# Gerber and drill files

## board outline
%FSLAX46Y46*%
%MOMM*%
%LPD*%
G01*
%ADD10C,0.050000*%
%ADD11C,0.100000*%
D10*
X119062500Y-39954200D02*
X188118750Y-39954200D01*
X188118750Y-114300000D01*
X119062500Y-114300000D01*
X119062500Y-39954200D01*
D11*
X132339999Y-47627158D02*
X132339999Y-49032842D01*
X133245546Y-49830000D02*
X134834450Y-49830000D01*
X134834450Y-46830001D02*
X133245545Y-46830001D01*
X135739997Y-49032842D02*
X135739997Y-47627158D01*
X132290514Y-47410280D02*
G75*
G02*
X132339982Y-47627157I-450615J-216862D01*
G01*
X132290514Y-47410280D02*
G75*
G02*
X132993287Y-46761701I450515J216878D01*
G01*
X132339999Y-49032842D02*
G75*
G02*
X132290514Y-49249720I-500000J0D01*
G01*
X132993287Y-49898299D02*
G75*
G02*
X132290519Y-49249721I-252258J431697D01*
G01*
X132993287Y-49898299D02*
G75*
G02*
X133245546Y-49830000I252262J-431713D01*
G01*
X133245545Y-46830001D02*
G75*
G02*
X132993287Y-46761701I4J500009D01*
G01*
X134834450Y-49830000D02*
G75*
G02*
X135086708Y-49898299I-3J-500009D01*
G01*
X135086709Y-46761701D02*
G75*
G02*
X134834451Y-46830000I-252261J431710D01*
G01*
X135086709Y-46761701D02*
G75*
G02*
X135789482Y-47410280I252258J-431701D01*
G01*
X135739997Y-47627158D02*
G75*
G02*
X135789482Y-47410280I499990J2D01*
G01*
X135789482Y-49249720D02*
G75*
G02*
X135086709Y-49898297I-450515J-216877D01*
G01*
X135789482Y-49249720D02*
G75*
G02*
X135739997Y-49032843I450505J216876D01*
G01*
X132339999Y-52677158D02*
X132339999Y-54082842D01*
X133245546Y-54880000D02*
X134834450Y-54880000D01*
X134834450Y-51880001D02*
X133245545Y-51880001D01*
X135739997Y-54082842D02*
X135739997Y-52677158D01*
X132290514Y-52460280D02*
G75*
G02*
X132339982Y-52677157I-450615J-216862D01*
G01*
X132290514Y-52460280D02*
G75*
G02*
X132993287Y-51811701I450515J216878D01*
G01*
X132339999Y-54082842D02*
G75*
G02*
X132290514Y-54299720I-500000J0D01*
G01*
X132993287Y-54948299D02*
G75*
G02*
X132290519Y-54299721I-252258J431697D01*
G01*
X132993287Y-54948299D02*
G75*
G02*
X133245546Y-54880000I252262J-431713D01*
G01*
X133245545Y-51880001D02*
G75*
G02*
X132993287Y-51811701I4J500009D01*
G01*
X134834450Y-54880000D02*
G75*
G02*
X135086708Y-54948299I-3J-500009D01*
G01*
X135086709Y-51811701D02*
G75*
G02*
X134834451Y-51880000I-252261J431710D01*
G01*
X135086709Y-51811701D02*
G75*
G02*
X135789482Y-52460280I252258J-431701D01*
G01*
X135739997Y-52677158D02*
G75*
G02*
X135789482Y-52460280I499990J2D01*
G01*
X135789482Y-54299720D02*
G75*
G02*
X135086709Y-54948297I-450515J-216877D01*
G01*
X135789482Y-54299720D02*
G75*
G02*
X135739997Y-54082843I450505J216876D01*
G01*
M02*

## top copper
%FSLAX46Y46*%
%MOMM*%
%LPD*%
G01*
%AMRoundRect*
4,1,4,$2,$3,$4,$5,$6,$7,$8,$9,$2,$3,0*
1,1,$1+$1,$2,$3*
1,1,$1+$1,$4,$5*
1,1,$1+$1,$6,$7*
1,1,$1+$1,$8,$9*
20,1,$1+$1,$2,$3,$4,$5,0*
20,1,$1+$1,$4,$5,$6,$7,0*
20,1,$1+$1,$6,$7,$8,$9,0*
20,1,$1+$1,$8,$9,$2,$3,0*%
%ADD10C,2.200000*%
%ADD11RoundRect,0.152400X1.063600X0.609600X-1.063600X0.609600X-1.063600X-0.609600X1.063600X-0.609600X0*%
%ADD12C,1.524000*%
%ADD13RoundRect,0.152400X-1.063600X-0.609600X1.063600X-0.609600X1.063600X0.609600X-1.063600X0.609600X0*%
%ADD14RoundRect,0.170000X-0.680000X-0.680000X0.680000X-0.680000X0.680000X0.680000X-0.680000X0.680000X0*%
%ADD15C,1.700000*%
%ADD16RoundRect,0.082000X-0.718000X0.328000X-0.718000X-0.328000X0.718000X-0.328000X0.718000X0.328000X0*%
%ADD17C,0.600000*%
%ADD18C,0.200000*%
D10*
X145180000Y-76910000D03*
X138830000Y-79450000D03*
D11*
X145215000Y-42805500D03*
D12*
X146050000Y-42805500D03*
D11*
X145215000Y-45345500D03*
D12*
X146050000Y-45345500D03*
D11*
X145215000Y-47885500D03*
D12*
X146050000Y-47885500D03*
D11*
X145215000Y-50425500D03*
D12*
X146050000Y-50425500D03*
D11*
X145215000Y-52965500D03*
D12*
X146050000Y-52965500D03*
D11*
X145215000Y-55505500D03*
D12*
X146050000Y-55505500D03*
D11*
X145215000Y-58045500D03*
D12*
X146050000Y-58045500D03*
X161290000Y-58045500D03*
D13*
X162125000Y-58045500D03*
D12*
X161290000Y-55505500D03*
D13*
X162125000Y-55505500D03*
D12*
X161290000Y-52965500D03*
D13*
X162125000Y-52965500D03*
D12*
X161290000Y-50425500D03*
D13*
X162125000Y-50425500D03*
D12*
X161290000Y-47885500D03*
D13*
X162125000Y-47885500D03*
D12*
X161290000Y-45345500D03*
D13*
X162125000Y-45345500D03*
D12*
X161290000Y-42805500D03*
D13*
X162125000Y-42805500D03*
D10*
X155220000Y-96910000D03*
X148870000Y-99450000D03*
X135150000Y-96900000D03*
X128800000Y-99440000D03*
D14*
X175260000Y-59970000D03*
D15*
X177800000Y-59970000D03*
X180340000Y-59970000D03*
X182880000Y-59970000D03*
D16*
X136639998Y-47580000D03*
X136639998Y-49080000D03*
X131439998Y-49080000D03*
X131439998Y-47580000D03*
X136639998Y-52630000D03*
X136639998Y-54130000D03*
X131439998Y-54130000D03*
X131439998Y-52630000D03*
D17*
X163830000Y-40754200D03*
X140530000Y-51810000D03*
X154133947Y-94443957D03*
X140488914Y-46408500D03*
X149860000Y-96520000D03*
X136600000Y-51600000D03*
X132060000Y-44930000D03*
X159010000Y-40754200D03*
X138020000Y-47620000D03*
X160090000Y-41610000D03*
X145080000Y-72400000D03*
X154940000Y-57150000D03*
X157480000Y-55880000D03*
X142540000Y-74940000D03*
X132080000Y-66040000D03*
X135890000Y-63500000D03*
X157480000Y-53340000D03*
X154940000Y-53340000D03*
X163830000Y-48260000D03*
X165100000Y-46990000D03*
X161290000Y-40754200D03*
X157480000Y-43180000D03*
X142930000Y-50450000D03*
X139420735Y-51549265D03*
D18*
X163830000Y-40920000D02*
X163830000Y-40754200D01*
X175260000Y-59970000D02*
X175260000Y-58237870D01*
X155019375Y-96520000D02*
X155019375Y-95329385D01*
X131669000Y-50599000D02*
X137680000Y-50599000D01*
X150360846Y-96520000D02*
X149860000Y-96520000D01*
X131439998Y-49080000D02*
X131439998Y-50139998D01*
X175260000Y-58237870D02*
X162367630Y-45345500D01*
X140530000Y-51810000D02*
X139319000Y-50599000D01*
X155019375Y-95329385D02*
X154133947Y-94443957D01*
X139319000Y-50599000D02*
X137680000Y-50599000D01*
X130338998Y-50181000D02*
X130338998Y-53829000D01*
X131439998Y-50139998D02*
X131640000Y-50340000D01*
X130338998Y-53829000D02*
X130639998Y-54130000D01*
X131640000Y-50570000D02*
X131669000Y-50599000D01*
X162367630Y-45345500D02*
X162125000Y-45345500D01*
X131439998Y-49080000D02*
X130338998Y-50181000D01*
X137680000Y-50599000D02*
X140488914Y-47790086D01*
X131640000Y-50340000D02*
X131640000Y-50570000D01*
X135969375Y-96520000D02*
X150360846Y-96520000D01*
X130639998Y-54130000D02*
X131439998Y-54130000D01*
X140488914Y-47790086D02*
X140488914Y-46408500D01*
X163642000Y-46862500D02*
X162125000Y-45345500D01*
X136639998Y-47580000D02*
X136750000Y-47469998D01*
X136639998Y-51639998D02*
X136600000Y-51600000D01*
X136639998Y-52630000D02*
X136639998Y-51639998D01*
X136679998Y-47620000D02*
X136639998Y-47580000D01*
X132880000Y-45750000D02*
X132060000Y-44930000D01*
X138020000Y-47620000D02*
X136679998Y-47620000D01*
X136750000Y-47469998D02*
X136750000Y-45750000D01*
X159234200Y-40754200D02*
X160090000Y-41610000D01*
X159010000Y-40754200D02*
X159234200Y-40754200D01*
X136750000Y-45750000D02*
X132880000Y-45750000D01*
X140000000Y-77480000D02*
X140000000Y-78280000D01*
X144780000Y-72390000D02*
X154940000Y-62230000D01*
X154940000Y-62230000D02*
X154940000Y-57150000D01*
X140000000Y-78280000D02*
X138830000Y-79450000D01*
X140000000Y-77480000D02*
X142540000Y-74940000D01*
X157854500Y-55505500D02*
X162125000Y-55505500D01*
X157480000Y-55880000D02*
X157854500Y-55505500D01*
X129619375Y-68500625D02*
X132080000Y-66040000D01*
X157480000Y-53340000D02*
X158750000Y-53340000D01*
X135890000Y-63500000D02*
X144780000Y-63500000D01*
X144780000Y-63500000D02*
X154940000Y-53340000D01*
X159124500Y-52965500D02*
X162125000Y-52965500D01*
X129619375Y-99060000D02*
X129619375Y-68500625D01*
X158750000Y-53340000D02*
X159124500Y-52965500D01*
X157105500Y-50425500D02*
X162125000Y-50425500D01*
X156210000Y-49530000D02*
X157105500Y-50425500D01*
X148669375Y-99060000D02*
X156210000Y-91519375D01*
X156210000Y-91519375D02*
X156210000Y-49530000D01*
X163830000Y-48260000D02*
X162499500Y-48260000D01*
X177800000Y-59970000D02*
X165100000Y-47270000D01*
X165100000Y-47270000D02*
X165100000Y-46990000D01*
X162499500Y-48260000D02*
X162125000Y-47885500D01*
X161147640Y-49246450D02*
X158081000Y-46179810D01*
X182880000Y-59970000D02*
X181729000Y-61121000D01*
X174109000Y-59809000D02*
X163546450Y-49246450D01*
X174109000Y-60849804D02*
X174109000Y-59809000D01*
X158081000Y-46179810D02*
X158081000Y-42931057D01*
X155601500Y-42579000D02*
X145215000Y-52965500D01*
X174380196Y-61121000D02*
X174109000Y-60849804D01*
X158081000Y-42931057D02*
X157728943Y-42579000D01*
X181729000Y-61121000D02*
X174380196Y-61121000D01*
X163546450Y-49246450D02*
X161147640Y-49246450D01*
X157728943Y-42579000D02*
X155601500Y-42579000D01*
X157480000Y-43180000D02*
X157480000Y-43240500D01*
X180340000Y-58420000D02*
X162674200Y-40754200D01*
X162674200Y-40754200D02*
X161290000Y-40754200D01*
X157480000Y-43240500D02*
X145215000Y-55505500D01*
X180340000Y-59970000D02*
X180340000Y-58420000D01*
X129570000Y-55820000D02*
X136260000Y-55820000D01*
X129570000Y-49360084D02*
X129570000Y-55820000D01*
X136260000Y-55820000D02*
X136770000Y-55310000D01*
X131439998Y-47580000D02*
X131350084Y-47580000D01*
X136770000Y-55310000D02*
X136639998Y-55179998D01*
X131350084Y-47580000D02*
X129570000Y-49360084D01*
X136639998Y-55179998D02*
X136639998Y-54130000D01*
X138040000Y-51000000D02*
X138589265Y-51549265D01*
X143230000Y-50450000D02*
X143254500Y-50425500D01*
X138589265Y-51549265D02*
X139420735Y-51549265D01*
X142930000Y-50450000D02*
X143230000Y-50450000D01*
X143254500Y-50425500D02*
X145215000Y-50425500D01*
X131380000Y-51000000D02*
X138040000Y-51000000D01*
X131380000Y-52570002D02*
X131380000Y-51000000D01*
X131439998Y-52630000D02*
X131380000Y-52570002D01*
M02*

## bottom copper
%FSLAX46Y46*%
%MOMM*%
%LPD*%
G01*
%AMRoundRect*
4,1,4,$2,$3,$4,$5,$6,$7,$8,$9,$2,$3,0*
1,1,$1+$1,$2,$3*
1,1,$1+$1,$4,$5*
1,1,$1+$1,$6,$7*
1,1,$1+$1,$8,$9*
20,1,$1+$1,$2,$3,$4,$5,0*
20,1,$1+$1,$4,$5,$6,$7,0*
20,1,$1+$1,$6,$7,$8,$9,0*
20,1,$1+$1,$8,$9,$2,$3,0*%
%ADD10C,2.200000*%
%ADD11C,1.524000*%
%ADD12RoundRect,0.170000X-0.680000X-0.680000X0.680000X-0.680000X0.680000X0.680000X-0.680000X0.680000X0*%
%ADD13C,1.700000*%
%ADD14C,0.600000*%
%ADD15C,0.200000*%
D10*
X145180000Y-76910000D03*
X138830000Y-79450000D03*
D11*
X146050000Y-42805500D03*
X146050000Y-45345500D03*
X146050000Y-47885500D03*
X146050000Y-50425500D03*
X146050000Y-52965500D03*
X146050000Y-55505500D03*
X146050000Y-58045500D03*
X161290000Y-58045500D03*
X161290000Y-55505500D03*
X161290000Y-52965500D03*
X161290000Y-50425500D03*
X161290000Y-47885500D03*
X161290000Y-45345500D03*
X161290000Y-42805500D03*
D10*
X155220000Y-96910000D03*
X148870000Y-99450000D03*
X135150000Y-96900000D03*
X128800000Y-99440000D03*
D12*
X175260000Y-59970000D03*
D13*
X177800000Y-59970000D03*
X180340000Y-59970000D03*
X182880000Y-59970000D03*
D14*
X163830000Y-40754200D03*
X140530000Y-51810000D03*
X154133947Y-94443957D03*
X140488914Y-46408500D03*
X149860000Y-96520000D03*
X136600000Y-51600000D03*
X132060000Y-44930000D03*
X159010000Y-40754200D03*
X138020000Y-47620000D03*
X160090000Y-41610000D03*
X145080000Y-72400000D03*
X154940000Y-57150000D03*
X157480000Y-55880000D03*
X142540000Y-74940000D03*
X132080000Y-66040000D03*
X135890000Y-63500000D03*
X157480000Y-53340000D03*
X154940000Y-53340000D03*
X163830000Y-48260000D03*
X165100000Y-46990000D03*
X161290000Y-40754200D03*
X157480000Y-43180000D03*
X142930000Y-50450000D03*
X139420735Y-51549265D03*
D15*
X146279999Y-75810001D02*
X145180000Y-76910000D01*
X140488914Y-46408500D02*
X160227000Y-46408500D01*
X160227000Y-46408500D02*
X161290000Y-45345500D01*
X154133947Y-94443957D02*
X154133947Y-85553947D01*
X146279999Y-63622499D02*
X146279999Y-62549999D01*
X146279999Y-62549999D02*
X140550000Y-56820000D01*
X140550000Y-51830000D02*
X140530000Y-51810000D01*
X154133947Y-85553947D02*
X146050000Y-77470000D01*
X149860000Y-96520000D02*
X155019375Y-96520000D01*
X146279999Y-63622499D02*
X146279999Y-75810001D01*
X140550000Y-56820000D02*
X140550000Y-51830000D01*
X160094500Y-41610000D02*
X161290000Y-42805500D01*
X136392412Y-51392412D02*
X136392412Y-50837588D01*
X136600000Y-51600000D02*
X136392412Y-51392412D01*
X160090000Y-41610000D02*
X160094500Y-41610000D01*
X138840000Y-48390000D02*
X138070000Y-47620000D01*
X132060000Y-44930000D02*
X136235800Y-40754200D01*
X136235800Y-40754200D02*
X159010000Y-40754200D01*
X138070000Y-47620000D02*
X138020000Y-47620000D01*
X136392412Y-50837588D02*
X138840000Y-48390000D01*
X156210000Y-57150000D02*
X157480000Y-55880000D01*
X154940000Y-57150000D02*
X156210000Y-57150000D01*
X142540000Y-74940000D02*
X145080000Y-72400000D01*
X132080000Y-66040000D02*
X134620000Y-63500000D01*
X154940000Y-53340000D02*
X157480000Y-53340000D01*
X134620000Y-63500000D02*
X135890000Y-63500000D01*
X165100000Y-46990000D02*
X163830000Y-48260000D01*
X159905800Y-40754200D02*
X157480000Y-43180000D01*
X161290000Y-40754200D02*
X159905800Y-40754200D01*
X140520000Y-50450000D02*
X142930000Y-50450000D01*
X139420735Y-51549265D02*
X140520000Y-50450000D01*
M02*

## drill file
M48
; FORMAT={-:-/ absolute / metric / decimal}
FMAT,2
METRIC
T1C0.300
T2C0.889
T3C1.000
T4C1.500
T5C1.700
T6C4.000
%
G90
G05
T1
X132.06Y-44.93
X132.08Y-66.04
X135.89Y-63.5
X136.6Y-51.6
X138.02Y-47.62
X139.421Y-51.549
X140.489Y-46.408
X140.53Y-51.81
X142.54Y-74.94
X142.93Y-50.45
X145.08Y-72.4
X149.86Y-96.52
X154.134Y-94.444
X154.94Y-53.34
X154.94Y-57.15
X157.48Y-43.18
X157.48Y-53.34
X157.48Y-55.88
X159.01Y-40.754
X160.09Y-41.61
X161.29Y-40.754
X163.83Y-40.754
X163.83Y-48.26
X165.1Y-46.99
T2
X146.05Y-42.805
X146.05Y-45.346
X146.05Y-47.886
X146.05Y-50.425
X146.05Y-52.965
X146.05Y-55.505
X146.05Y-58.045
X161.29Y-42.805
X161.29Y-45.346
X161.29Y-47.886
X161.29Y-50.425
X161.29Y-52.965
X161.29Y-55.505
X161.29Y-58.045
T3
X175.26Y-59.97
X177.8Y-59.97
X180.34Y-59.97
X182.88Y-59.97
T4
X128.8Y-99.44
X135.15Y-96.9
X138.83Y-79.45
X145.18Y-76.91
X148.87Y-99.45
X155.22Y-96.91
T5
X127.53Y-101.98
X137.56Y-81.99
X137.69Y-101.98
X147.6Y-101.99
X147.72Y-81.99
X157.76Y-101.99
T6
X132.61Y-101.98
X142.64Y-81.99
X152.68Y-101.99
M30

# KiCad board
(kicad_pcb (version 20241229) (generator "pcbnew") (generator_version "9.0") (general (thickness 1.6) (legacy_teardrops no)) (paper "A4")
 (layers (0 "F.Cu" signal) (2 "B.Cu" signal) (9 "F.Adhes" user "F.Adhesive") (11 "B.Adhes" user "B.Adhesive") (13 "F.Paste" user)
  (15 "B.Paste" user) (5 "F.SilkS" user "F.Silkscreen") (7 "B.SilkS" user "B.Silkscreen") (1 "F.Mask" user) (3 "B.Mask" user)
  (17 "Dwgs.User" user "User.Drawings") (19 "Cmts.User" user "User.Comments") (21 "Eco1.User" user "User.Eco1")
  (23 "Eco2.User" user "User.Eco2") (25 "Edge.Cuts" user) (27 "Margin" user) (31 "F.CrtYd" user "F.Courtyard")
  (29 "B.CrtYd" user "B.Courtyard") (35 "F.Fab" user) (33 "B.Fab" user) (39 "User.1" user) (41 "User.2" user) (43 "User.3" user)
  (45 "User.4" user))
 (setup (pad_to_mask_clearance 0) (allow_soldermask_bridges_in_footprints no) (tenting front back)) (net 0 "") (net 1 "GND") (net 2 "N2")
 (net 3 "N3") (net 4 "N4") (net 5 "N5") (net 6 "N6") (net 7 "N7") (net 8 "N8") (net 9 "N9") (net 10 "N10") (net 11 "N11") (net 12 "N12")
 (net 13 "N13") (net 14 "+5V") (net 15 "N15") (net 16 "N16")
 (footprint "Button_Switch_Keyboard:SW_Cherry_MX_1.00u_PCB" (layer "F.Cu") (at 145.18 76.91)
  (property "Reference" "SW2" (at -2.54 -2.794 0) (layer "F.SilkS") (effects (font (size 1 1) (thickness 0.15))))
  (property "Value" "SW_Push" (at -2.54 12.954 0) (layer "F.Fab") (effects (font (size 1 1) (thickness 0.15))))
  (pad "" np_thru_hole circle (at -7.62 5.08) (size 1.7 1.7) (drill 1.7) (layers "*.Cu" "*.Mask"))
  (pad "" np_thru_hole circle (at -2.54 5.08) (size 4 4) (drill 4) (layers "*.Cu" "*.Mask"))
  (pad "" np_thru_hole circle (at 2.54 5.08) (size 1.7 1.7) (drill 1.7) (layers "*.Cu" "*.Mask"))
  (pad "1" thru_hole circle (at 0 0) (size 2.2 2.2) (drill 1.5) (layers "*.Cu" "*.Mask") (remove_unused_layers no) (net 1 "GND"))
  (pad "2" thru_hole circle (at -6.35 2.54) (size 2.2 2.2) (drill 1.5) (layers "*.Cu" "*.Mask") (remove_unused_layers no) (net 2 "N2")))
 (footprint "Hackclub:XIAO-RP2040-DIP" (layer "F.Cu") (at 153.67 50.4255)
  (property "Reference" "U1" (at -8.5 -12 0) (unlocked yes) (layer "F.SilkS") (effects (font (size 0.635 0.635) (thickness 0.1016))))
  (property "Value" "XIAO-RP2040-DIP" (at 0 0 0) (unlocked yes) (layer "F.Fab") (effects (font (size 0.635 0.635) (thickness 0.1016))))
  (pad "1" smd roundrect (at -8.455 -7.62 180) (size 2.432 1.524) (layers "F.Cu" "F.Mask") (roundrect_rratio 0.1) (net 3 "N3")
   (thermal_bridge_angle 45))
  (pad "1" thru_hole circle (at -7.62 -7.62 180) (size 1.524 1.524) (drill 0.889) (layers "*.Cu" "*.Mask") (remove_unused_layers no)
   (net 3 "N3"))
  (pad "2" smd roundrect (at -8.455 -5.08 180) (size 2.432 1.524) (layers "F.Cu" "F.Mask") (roundrect_rratio 0.1) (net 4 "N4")
   (thermal_bridge_angle 45))
  (pad "2" thru_hole circle (at -7.62 -5.08 180) (size 1.524 1.524) (drill 0.889) (layers "*.Cu" "*.Mask") (remove_unused_layers no)
   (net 4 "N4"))
  (pad "3" smd roundrect (at -8.455 -2.54 180) (size 2.432 1.524) (layers "F.Cu" "F.Mask") (roundrect_rratio 0.1) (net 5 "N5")
   (thermal_bridge_angle 45))
  (pad "3" thru_hole circle (at -7.62 -2.54 180) (size 1.524 1.524) (drill 0.889) (layers "*.Cu" "*.Mask") (remove_unused_layers no)
   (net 5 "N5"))
  (pad "4" smd roundrect (at -8.455 0 180) (size 2.432 1.524) (layers "F.Cu" "F.Mask") (roundrect_rratio 0.1) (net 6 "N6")
   (thermal_bridge_angle 45))
  (pad "4" thru_hole circle (at -7.62 0 180) (size 1.524 1.524) (drill 0.889) (layers "*.Cu" "*.Mask") (remove_unused_layers no)
   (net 6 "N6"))
  (pad "5" smd roundrect (at -8.455 2.54 180) (size 2.432 1.524) (layers "F.Cu" "F.Mask") (roundrect_rratio 0.1) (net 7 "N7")
   (thermal_bridge_angle 45))
  (pad "5" thru_hole circle (at -7.62 2.54 180) (size 1.524 1.524) (drill 0.889) (layers "*.Cu" "*.Mask") (remove_unused_layers no)
   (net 7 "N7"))
  (pad "6" smd roundrect (at -8.455 5.08 180) (size 2.432 1.524) (layers "F.Cu" "F.Mask") (roundrect_rratio 0.1) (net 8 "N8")
   (thermal_bridge_angle 45))
  (pad "6" thru_hole circle (at -7.62 5.08 180) (size 1.524 1.524) (drill 0.889) (layers "*.Cu" "*.Mask") (remove_unused_layers no)
   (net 8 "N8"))
  (pad "7" smd roundrect (at -8.455 7.62 180) (size 2.432 1.524) (layers "F.Cu" "F.Mask") (roundrect_rratio 0.1) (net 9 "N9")
   (thermal_bridge_angle 45))
  (pad "7" thru_hole circle (at -7.62 7.62 180) (size 1.524 1.524) (drill 0.889) (layers "*.Cu" "*.Mask") (remove_unused_layers no)
   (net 9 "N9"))
  (pad "8" thru_hole circle (at 7.62 7.62) (size 1.524 1.524) (drill 0.889) (layers "*.Cu" "*.Mask") (remove_unused_layers no)
   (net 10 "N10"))
  (pad "8" smd roundrect (at 8.455 7.62) (size 2.432 1.524) (layers "F.Cu" "F.Mask") (roundrect_rratio 0.1) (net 10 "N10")
   (thermal_bridge_angle 45))
  (pad "9" thru_hole circle (at 7.62 5.08) (size 1.524 1.524) (drill 0.889) (layers "*.Cu" "*.Mask") (remove_unused_layers no) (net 2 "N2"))
  (pad "9" smd roundrect (at 8.455 5.08) (size 2.432 1.524) (layers "F.Cu" "F.Mask") (roundrect_rratio 0.1) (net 2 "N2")
   (thermal_bridge_angle 45))
  (pad "10" thru_hole circle (at 7.62 2.54) (size 1.524 1.524) (drill 0.889) (layers "*.Cu" "*.Mask") (remove_unused_layers no)
   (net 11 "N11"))
  (pad "10" smd roundrect (at 8.455 2.54) (size 2.432 1.524) (layers "F.Cu" "F.Mask") (roundrect_rratio 0.1) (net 11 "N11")
   (thermal_bridge_angle 45))
  (pad "11" thru_hole circle (at 7.62 0) (size 1.524 1.524) (drill 0.889) (layers "*.Cu" "*.Mask") (remove_unused_layers no) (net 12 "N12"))
  (pad "11" smd roundrect (at 8.455 0) (size 2.432 1.524) (layers "F.Cu" "F.Mask") (roundrect_rratio 0.1) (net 12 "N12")
   (thermal_bridge_angle 45))
  (pad "12" thru_hole circle (at 7.62 -2.54) (size 1.524 1.524) (drill 0.889) (layers "*.Cu" "*.Mask") (remove_unused_layers no)
   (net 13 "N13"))
  (pad "12" smd roundrect (at 8.455 -2.54) (size 2.432 1.524) (layers "F.Cu" "F.Mask") (roundrect_rratio 0.1) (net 13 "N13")
   (thermal_bridge_angle 45))
  (pad "13" thru_hole circle (at 7.62 -5.08) (size 1.524 1.524) (drill 0.889) (layers "*.Cu" "*.Mask") (remove_unused_layers no)
   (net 1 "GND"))
  (pad "13" smd roundrect (at 8.455 -5.08) (size 2.432 1.524) (layers "F.Cu" "F.Mask") (roundrect_rratio 0.1) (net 1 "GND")
   (thermal_bridge_angle 45))
  (pad "14" thru_hole circle (at 7.62 -7.62) (size 1.524 1.524) (drill 0.889) (layers "*.Cu" "*.Mask") (remove_unused_layers no)
   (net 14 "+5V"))
  (pad "14" smd roundrect (at 8.455 -7.62) (size 2.432 1.524) (layers "F.Cu" "F.Mask") (roundrect_rratio 0.1) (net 14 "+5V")
   (thermal_bridge_angle 45)))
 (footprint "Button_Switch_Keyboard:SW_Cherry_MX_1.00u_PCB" (layer "F.Cu") (at 155.22 96.91)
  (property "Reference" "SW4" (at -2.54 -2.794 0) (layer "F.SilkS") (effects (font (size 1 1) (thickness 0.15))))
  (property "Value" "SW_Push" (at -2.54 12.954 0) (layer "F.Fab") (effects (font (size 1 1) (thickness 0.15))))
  (pad "" np_thru_hole circle (at -7.62 5.08) (size 1.7 1.7) (drill 1.7) (layers "*.Cu" "*.Mask"))
  (pad "" np_thru_hole circle (at -2.54 5.08) (size 4 4) (drill 4) (layers "*.Cu" "*.Mask"))
  (pad "" np_thru_hole circle (at 2.54 5.08) (size 1.7 1.7) (drill 1.7) (layers "*.Cu" "*.Mask"))
  (pad "1" thru_hole circle (at 0 0) (size 2.2 2.2) (drill 1.5) (layers "*.Cu" "*.Mask") (remove_unused_layers no) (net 1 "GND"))
  (pad "2" thru_hole circle (at -6.35 2.54) (size 2.2 2.2) (drill 1.5) (layers "*.Cu" "*.Mask") (remove_unused_layers no) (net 12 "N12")))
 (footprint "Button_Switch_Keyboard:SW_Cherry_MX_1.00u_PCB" (layer "F.Cu") (at 135.15 96.9)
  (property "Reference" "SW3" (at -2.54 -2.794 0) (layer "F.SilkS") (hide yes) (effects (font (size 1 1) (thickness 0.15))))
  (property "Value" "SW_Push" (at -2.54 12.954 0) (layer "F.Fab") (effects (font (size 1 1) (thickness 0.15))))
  (pad "" np_thru_hole circle (at -7.62 5.08) (size 1.7 1.7) (drill 1.7) (layers "*.Cu" "*.Mask"))
  (pad "" np_thru_hole circle (at -2.54 5.08) (size 4 4) (drill 4) (layers "*.Cu" "*.Mask"))
  (pad "" np_thru_hole circle (at 2.54 5.08) (size 1.7 1.7) (drill 1.7) (layers "*.Cu" "*.Mask"))
  (pad "1" thru_hole circle (at 0 0) (size 2.2 2.2) (drill 1.5) (layers "*.Cu" "*.Mask") (remove_unused_layers no) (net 1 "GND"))
  (pad "2" thru_hole circle (at -6.35 2.54) (size 2.2 2.2) (drill 1.5) (layers "*.Cu" "*.Mask") (remove_unused_layers no) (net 11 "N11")))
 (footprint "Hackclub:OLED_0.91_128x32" (layer "F.Cu") (at 175.26 59.97)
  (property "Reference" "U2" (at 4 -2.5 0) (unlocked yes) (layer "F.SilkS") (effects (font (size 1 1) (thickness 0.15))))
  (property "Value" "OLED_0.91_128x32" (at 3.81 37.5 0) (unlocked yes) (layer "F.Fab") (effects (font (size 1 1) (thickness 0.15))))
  (pad "1" thru_hole roundrect (at 0 0) (size 1.7 1.7) (drill 1) (layers "*.Cu" "*.Mask") (remove_unused_layers no) (roundrect_rratio 0.1)
   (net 1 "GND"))
  (pad "2" thru_hole circle (at 2.54 0) (size 1.7 1.7) (drill 1) (layers "*.Cu" "*.Mask") (remove_unused_layers no) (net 13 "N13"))
  (pad "3" thru_hole circle (at 5.08 0) (size 1.7 1.7) (drill 1) (layers "*.Cu" "*.Mask") (remove_unused_layers no) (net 8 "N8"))
  (pad "4" thru_hole circle (at 7.62 0) (size 1.7 1.7) (drill 1) (layers "*.Cu" "*.Mask") (remove_unused_layers no) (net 7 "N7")))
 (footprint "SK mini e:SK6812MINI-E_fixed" (layer "B.Cu") (at 134.039999 48.432842 180)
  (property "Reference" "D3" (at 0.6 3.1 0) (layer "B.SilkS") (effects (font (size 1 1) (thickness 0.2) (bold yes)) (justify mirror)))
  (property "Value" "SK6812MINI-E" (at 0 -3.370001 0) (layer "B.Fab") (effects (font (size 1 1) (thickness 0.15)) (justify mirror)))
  (fp_line (start 1.7 0.805684) (end 1.7 -0.6) (stroke (width 0.1) (type solid)) (layer "Edge.Cuts"))
  (fp_line (start 0.794453 -1.397158) (end -0.794451 -1.397158) (stroke (width 0.1) (type solid)) (layer "Edge.Cuts"))
  (fp_line (start -0.794451 1.602841) (end 0.794454 1.602841) (stroke (width 0.1) (type solid)) (layer "Edge.Cuts"))
  (fp_line (start -1.699998 -0.6) (end -1.699998 0.805684) (stroke (width 0.1) (type solid)) (layer "Edge.Cuts"))
  (fp_arc (start 1.749485 1.022562) (mid 1.712532 0.91691) (end 1.7 0.805685) (stroke (width 0.1) (type solid)) (layer "Edge.Cuts"))
  (fp_arc (start 1.749485 1.022562) (mid 1.638072 1.606877) (end 1.046712 1.67114) (stroke (width 0.1) (type solid)) (layer "Edge.Cuts"))
  (fp_arc (start 1.7 -0.6) (mid 1.712528 -0.711226) (end 1.749485 -0.816878) (stroke (width 0.1) (type solid)) (layer "Edge.Cuts"))
  (fp_arc (start 1.046712 -1.465457) (mid 1.638073 -1.401193) (end 1.749485 -0.816877) (stroke (width 0.1) (type solid)) (layer "Edge.Cuts"))
  (fp_arc (start 1.046712 -1.465457) (mid 0.925124 -1.414535) (end 0.794453 -1.397158) (stroke (width 0.1) (type solid)) (layer "Edge.Cuts"))
  (fp_arc (start 0.794454 1.602841) (mid 0.925124 1.620218) (end 1.046712 1.67114) (stroke (width 0.1) (type solid)) (layer "Edge.Cuts"))
  (fp_arc (start -0.794451 -1.397158) (mid -0.925121 -1.414535) (end -1.046709 -1.465457) (stroke (width 0.1) (type solid))
   (layer "Edge.Cuts"))
  (fp_arc (start -1.04671 1.671141) (mid -0.925122 1.620219) (end -0.794452 1.602842) (stroke (width 0.1) (type solid)) (layer "Edge.Cuts"))
  (fp_arc (start -1.04671 1.671141) (mid -1.63807 1.606877) (end -1.749483 1.022562) (stroke (width 0.1) (type solid)) (layer "Edge.Cuts"))
  (fp_arc (start -1.699998 0.805684) (mid -1.712526 0.91691) (end -1.749483 1.022562) (stroke (width 0.1) (type solid)) (layer "Edge.Cuts"))
  (fp_arc (start -1.749483 -0.816878) (mid -1.638069 -1.401192) (end -1.04671 -1.465455) (stroke (width 0.1) (type solid))
   (layer "Edge.Cuts"))
  (fp_arc (start -1.749483 -0.816878) (mid -1.712526 -0.711226) (end -1.699998 -0.600001) (stroke (width 0.1) (type solid))
   (layer "Edge.Cuts"))
  (pad "1" smd roundrect (at -2.599999 0.852842 270) (size 0.82 1.6) (layers "F.Cu" "F.Mask" "F.Paste") (roundrect_rratio 0.1)
   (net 14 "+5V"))
  (pad "2" smd roundrect (at -2.599999 -0.647158 270) (size 0.82 1.6) (layers "F.Cu" "F.Mask" "F.Paste") (roundrect_rratio 0.1)
   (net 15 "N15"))
  (pad "3" smd roundrect (at 2.600001 -0.647158 270) (size 0.82 1.6) (layers "F.Cu" "F.Mask" "F.Paste") (roundrect_rratio 0.1) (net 1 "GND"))
  (pad "4" smd roundrect (at 2.600001 0.852842 270) (size 0.82 1.6) (layers "F.Cu" "F.Mask" "F.Paste") (roundrect_rratio 0.1) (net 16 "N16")))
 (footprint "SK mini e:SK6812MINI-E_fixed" (layer "B.Cu") (at 134.039999 53.482842 180)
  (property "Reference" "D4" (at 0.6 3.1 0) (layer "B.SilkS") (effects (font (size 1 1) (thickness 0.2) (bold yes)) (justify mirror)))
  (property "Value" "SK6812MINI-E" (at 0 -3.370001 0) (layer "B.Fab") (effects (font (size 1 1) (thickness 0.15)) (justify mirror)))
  (fp_line (start 1.7 0.805684) (end 1.7 -0.6) (stroke (width 0.1) (type solid)) (layer "Edge.Cuts"))
  (fp_line (start 0.794453 -1.397158) (end -0.794451 -1.397158) (stroke (width 0.1) (type solid)) (layer "Edge.Cuts"))
  (fp_line (start -0.794451 1.602841) (end 0.794454 1.602841) (stroke (width 0.1) (type solid)) (layer "Edge.Cuts"))
  (fp_line (start -1.699998 -0.6) (end -1.699998 0.805684) (stroke (width 0.1) (type solid)) (layer "Edge.Cuts"))
  (fp_arc (start 1.749485 1.022562) (mid 1.712532 0.91691) (end 1.7 0.805685) (stroke (width 0.1) (type solid)) (layer "Edge.Cuts"))
  (fp_arc (start 1.749485 1.022562) (mid 1.638072 1.606877) (end 1.046712 1.67114) (stroke (width 0.1) (type solid)) (layer "Edge.Cuts"))
  (fp_arc (start 1.7 -0.6) (mid 1.712528 -0.711226) (end 1.749485 -0.816878) (stroke (width 0.1) (type solid)) (layer "Edge.Cuts"))
  (fp_arc (start 1.046712 -1.465457) (mid 1.638073 -1.401193) (end 1.749485 -0.816877) (stroke (width 0.1) (type solid)) (layer "Edge.Cuts"))
  (fp_arc (start 1.046712 -1.465457) (mid 0.925124 -1.414535) (end 0.794453 -1.397158) (stroke (width 0.1) (type solid)) (layer "Edge.Cuts"))
  (fp_arc (start 0.794454 1.602841) (mid 0.925124 1.620218) (end 1.046712 1.67114) (stroke (width 0.1) (type solid)) (layer "Edge.Cuts"))
  (fp_arc (start -0.794451 -1.397158) (mid -0.925121 -1.414535) (end -1.046709 -1.465457) (stroke (width 0.1) (type solid))
   (layer "Edge.Cuts"))
  (fp_arc (start -1.04671 1.671141) (mid -0.925122 1.620219) (end -0.794452 1.602842) (stroke (width 0.1) (type solid)) (layer "Edge.Cuts"))
  (fp_arc (start -1.04671 1.671141) (mid -1.63807 1.606877) (end -1.749483 1.022562) (stroke (width 0.1) (type solid)) (layer "Edge.Cuts"))
  (fp_arc (start -1.699998 0.805684) (mid -1.712526 0.91691) (end -1.749483 1.022562) (stroke (width 0.1) (type solid)) (layer "Edge.Cuts"))
  (fp_arc (start -1.749483 -0.816878) (mid -1.638069 -1.401192) (end -1.04671 -1.465455) (stroke (width 0.1) (type solid))
   (layer "Edge.Cuts"))
  (fp_arc (start -1.749483 -0.816878) (mid -1.712526 -0.711226) (end -1.699998 -0.600001) (stroke (width 0.1) (type solid))
   (layer "Edge.Cuts"))
  (pad "1" smd roundrect (at -2.599999 0.852842 270) (size 0.82 1.6) (layers "F.Cu" "F.Mask" "F.Paste") (roundrect_rratio 0.1)
   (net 14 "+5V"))
  (pad "2" smd roundrect (at -2.599999 -0.647158 270) (size 0.82 1.6) (layers "F.Cu" "F.Mask" "F.Paste") (roundrect_rratio 0.1)
   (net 16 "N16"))
  (pad "3" smd roundrect (at 2.600001 -0.647158 270) (size 0.82 1.6) (layers "F.Cu" "F.Mask" "F.Paste") (roundrect_rratio 0.1) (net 1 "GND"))
  (pad "4" smd roundrect (at 2.600001 0.852842 270) (size 0.82 1.6) (layers "F.Cu" "F.Mask" "F.Paste") (roundrect_rratio 0.1) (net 6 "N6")))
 (gr_rect (start 119.0625 39.9542) (end 188.11875 114.3) (stroke (width 0.05) (type default)) (fill no) (layer "Edge.Cuts"))
 (segment (start 163.83 40.92) (end 163.83 40.7542) (width 0.2) (layer "F.Cu") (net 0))
 (via (at 163.83 40.7542) (size 0.6) (drill 0.3) (layers "F.Cu" "B.Cu") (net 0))
 (segment (start 175.26 59.97) (end 175.26 58.23787) (width 0.2) (layer "F.Cu") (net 1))
 (segment (start 155.019375 96.52) (end 155.019375 95.329385) (width 0.2) (layer "F.Cu") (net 1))
 (segment (start 131.669 50.599) (end 137.68 50.599) (width 0.2) (layer "F.Cu") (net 1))
 (segment (start 150.360846 96.52) (end 149.86 96.52) (width 0.2) (layer "F.Cu") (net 1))
 (segment (start 131.439998 49.08) (end 131.439998 50.139998) (width 0.2) (layer "F.Cu") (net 1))
 (segment (start 175.26 58.23787) (end 162.36763 45.3455) (width 0.2) (layer "F.Cu") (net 1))
 (segment (start 140.53 51.81) (end 139.319 50.599) (width 0.2) (layer "F.Cu") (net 1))
 (segment (start 155.019375 95.329385) (end 154.133947 94.443957) (width 0.2) (layer "F.Cu") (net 1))
 (segment (start 139.319 50.599) (end 137.68 50.599) (width 0.2) (layer "F.Cu") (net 1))
 (segment (start 130.338998 50.181) (end 130.338998 53.829) (width 0.2) (layer "F.Cu") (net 1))
 (segment (start 131.439998 50.139998) (end 131.64 50.34) (width 0.2) (layer "F.Cu") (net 1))
 (segment (start 130.338998 53.829) (end 130.639998 54.13) (width 0.2) (layer "F.Cu") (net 1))
 (segment (start 131.64 50.57) (end 131.669 50.599) (width 0.2) (layer "F.Cu") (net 1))
 (segment (start 162.36763 45.3455) (end 162.125 45.3455) (width 0.2) (layer "F.Cu") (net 1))
 (segment (start 131.439998 49.08) (end 130.338998 50.181) (width 0.2) (layer "F.Cu") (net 1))
 (segment (start 137.68 50.599) (end 140.488914 47.790086) (width 0.2) (layer "F.Cu") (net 1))
 (segment (start 131.64 50.34) (end 131.64 50.57) (width 0.2) (layer "F.Cu") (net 1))
 (segment (start 135.969375 96.52) (end 150.360846 96.52) (width 0.2) (layer "F.Cu") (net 1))
 (segment (start 130.639998 54.13) (end 131.439998 54.13) (width 0.2) (layer "F.Cu") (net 1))
 (segment (start 140.488914 47.790086) (end 140.488914 46.4085) (width 0.2) (layer "F.Cu") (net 1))
 (segment (start 163.642 46.8625) (end 162.125 45.3455) (width 0.2) (layer "F.Cu") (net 1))
 (via (at 140.53 51.81) (size 0.6) (drill 0.3) (layers "F.Cu" "B.Cu") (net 1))
 (via (at 154.133947 94.443957) (size 0.6) (drill 0.3) (layers "F.Cu" "B.Cu") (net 1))
 (via (at 140.488914 46.4085) (size 0.6) (drill 0.3) (layers "F.Cu" "B.Cu") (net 1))
 (via (at 149.86 96.52) (size 0.6) (drill 0.3) (layers "F.Cu" "B.Cu") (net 1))
 (segment (start 146.279999 75.810001) (end 145.18 76.91) (width 0.2) (layer "B.Cu") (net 1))
 (segment (start 140.488914 46.4085) (end 160.227 46.4085) (width 0.2) (layer "B.Cu") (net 1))
 (segment (start 160.227 46.4085) (end 161.29 45.3455) (width 0.2) (layer "B.Cu") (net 1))
 (segment (start 154.133947 94.443957) (end 154.133947 85.553947) (width 0.2) (layer "B.Cu") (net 1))
 (segment (start 146.279999 63.622499) (end 146.279999 62.549999) (width 0.2) (layer "B.Cu") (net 1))
 (segment (start 146.279999 62.549999) (end 140.55 56.82) (width 0.2) (layer "B.Cu") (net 1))
 (segment (start 140.55 51.83) (end 140.53 51.81) (width 0.2) (layer "B.Cu") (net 1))
 (segment (start 154.133947 85.553947) (end 146.05 77.47) (width 0.2) (layer "B.Cu") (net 1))
 (segment (start 149.86 96.52) (end 155.019375 96.52) (width 0.2) (layer "B.Cu") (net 1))
 (segment (start 146.279999 63.622499) (end 146.279999 75.810001) (width 0.2) (layer "B.Cu") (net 1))
 (segment (start 140.55 56.82) (end 140.55 51.83) (width 0.2) (layer "B.Cu") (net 1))
 (segment (start 136.639998 47.58) (end 136.75 47.469998) (width 0.2) (layer "F.Cu") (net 14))
 (segment (start 136.639998 51.639998) (end 136.6 51.6) (width 0.2) (layer "F.Cu") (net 14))
 (segment (start 136.639998 52.63) (end 136.639998 51.639998) (width 0.2) (layer "F.Cu") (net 14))
 (segment (start 136.679998 47.62) (end 136.639998 47.58) (width 0.2) (layer "F.Cu") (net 14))
 (segment (start 132.88 45.75) (end 132.06 44.93) (width 0.2) (layer "F.Cu") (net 14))
 (segment (start 138.02 47.62) (end 136.679998 47.62) (width 0.2) (layer "F.Cu") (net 14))
 (segment (start 136.75 47.469998) (end 136.75 45.75) (width 0.2) (layer "F.Cu") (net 14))
 (segment (start 159.2342 40.7542) (end 160.09 41.61) (width 0.2) (layer "F.Cu") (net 14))
 (segment (start 159.01 40.7542) (end 159.2342 40.7542) (width 0.2) (layer "F.Cu") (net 14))
 (segment (start 136.75 45.75) (end 132.88 45.75) (width 0.2) (layer "F.Cu") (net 14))
 (via (at 136.6 51.6) (size 0.6) (drill 0.3) (layers "F.Cu" "B.Cu") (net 14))
 (via (at 132.06 44.93) (size 0.6) (drill 0.3) (layers "F.Cu" "B.Cu") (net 14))
 (via (at 159.01 40.7542) (size 0.6) (drill 0.3) (layers "F.Cu" "B.Cu") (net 14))
 (via (at 138.02 47.62) (size 0.6) (drill 0.3) (layers "F.Cu" "B.Cu") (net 14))
 (via (at 160.09 41.61) (size 0.6) (drill 0.3) (layers "F.Cu" "B.Cu") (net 14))
 (segment (start 160.0945 41.61) (end 161.29 42.8055) (width 0.2) (layer "B.Cu") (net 14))
 (segment (start 136.392412 51.392412) (end 136.392412 50.837588) (width 0.2) (layer "B.Cu") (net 14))
 (segment (start 136.6 51.6) (end 136.392412 51.392412) (width 0.2) (layer "B.Cu") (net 14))
 (segment (start 160.09 41.61) (end 160.0945 41.61) (width 0.2) (layer "B.Cu") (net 14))
 (segment (start 138.84 48.39) (end 138.07 47.62) (width 0.2) (layer "B.Cu") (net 14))
 (segment (start 132.06 44.93) (end 136.2358 40.7542) (width 0.2) (layer "B.Cu") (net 14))
 (segment (start 136.2358 40.7542) (end 159.01 40.7542) (width 0.2) (layer "B.Cu") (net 14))
 (segment (start 138.07 47.62) (end 138.02 47.62) (width 0.2) (layer "B.Cu") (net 14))
 (segment (start 136.392412 50.837588) (end 138.84 48.39) (width 0.2) (layer "B.Cu") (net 14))
 (segment (start 140 77.48) (end 140 78.28) (width 0.2) (layer "F.Cu") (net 2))
 (segment (start 144.78 72.39) (end 154.94 62.23) (width 0.2) (layer "F.Cu") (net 2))
 (segment (start 154.94 62.23) (end 154.94 57.15) (width 0.2) (layer "F.Cu") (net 2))
 (segment (start 140 78.28) (end 138.83 79.45) (width 0.2) (layer "F.Cu") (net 2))
 (segment (start 140 77.48) (end 142.54 74.94) (width 0.2) (layer "F.Cu") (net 2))
 (segment (start 157.8545 55.5055) (end 162.125 55.5055) (width 0.2) (layer "F.Cu") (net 2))
 (segment (start 157.48 55.88) (end 157.8545 55.5055) (width 0.2) (layer "F.Cu") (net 2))
 (via (at 145.08 72.4) (size 0.6) (drill 0.3) (layers "F.Cu" "B.Cu") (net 2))
 (via (at 154.94 57.15) (size 0.6) (drill 0.3) (layers "F.Cu" "B.Cu") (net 2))
 (via (at 157.48 55.88) (size 0.6) (drill 0.3) (layers "F.Cu" "B.Cu") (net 2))
 (via (at 142.54 74.94) (size 0.6) (drill 0.3) (layers "F.Cu" "B.Cu") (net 2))
 (segment (start 156.21 57.15) (end 157.48 55.88) (width 0.2) (layer "B.Cu") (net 2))
 (segment (start 154.94 57.15) (end 156.21 57.15) (width 0.2) (layer "B.Cu") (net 2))
 (segment (start 142.54 74.94) (end 145.08 72.4) (width 0.2) (layer "B.Cu") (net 2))
 (segment (start 129.619375 68.500625) (end 132.08 66.04) (width 0.2) (layer "F.Cu") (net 11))
 (segment (start 157.48 53.34) (end 158.75 53.34) (width 0.2) (layer "F.Cu") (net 11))
 (segment (start 135.89 63.5) (end 144.78 63.5) (width 0.2) (layer "F.Cu") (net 11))
 (segment (start 144.78 63.5) (end 154.94 53.34) (width 0.2) (layer "F.Cu") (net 11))
 (segment (start 159.1245 52.9655) (end 162.125 52.9655) (width 0.2) (layer "F.Cu") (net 11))
 (segment (start 129.619375 99.06) (end 129.619375 68.500625) (width 0.2) (layer "F.Cu") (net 11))
 (segment (start 158.75 53.34) (end 159.1245 52.9655) (width 0.2) (layer "F.Cu") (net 11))
 (via (at 132.08 66.04) (size 0.6) (drill 0.3) (layers "F.Cu" "B.Cu") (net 11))
 (via (at 135.89 63.5) (size 0.6) (drill 0.3) (layers "F.Cu" "B.Cu") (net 11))
 (via (at 157.48 53.34) (size 0.6) (drill 0.3) (layers "F.Cu" "B.Cu") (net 11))
 (via (at 154.94 53.34) (size 0.6) (drill 0.3) (layers "F.Cu" "B.Cu") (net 11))
 (segment (start 132.08 66.04) (end 134.62 63.5) (width 0.2) (layer "B.Cu") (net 11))
 (segment (start 154.94 53.34) (end 157.48 53.34) (width 0.2) (layer "B.Cu") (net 11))
 (segment (start 134.62 63.5) (end 135.89 63.5) (width 0.2) (layer "B.Cu") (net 11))
 (segment (start 157.1055 50.4255) (end 162.125 50.4255) (width 0.2) (layer "F.Cu") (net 12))
 (segment (start 156.21 49.53) (end 157.1055 50.4255) (width 0.2) (layer "F.Cu") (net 12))
 (segment (start 148.669375 99.06) (end 156.21 91.519375) (width 0.2) (layer "F.Cu") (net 12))
 (segment (start 156.21 91.519375) (end 156.21 49.53) (width 0.2) (layer "F.Cu") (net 12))
 (segment (start 163.83 48.26) (end 162.4995 48.26) (width 0.2) (layer "F.Cu") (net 13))
 (segment (start 177.8 59.97) (end 165.1 47.27) (width 0.2) (layer "F.Cu") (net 13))
 (segment (start 165.1 47.27) (end 165.1 46.99) (width 0.2) (layer "F.Cu") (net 13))
 (segment (start 162.4995 48.26) (end 162.125 47.8855) (width 0.2) (layer "F.Cu") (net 13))
 (via (at 163.83 48.26) (size 0.6) (drill 0.3) (layers "F.Cu" "B.Cu") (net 13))
 (via (at 165.1 46.99) (size 0.6) (drill 0.3) (layers "F.Cu" "B.Cu") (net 13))
 (segment (start 165.1 46.99) (end 163.83 48.26) (width 0.2) (layer "B.Cu") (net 13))
 (segment (start 161.14764 49.24645) (end 158.081 46.17981) (width 0.2) (layer "F.Cu") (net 7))
 (segment (start 182.88 59.97) (end 181.729 61.121) (width 0.2) (layer "F.Cu") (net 7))
 (segment (start 174.109 59.809) (end 163.54645 49.24645) (width 0.2) (layer "F.Cu") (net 7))
 (segment (start 174.109 60.849804) (end 174.109 59.809) (width 0.2) (layer "F.Cu") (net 7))
 (segment (start 158.081 46.17981) (end 158.081 42.931057) (width 0.2) (layer "F.Cu") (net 7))
 (segment (start 155.6015 42.579) (end 145.215 52.9655) (width 0.2) (layer "F.Cu") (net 7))
 (segment (start 174.380196 61.121) (end 174.109 60.849804) (width 0.2) (layer "F.Cu") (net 7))
 (segment (start 158.081 42.931057) (end 157.728943 42.579) (width 0.2) (layer "F.Cu") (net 7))
 (segment (start 181.729 61.121) (end 174.380196 61.121) (width 0.2) (layer "F.Cu") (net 7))
 (segment (start 163.54645 49.24645) (end 161.14764 49.24645) (width 0.2) (layer "F.Cu") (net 7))
 (segment (start 157.728943 42.579) (end 155.6015 42.579) (width 0.2) (layer "F.Cu") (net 7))
 (segment (start 157.48 43.18) (end 157.48 43.2405) (width 0.2) (layer "F.Cu") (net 8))
 (segment (start 180.34 58.42) (end 162.6742 40.7542) (width 0.2) (layer "F.Cu") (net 8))
 (segment (start 162.6742 40.7542) (end 161.29 40.7542) (width 0.2) (layer "F.Cu") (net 8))
 (segment (start 157.48 43.2405) (end 145.215 55.5055) (width 0.2) (layer "F.Cu") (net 8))
 (segment (start 180.34 59.97) (end 180.34 58.42) (width 0.2) (layer "F.Cu") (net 8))
 (via (at 161.29 40.7542) (size 0.6) (drill 0.3) (layers "F.Cu" "B.Cu") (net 8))
 (via (at 157.48 43.18) (size 0.6) (drill 0.3) (layers "F.Cu" "B.Cu") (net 8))
 (segment (start 159.9058 40.7542) (end 157.48 43.18) (width 0.2) (layer "B.Cu") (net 8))
 (segment (start 161.29 40.7542) (end 159.9058 40.7542) (width 0.2) (layer "B.Cu") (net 8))
 (segment (start 129.57 55.82) (end 136.26 55.82) (width 0.2) (layer "F.Cu") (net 16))
 (segment (start 129.57 49.360084) (end 129.57 55.82) (width 0.2) (layer "F.Cu") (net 16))
 (segment (start 136.26 55.82) (end 136.77 55.31) (width 0.2) (layer "F.Cu") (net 16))
 (segment (start 131.439998 47.58) (end 131.350084 47.58) (width 0.2) (layer "F.Cu") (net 16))
 (segment (start 136.77 55.31) (end 136.639998 55.179998) (width 0.2) (layer "F.Cu") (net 16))
 (segment (start 131.350084 47.58) (end 129.57 49.360084) (width 0.2) (layer "F.Cu") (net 16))
 (segment (start 136.639998 55.179998) (end 136.639998 54.13) (width 0.2) (layer "F.Cu") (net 16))
 (segment (start 138.04 51) (end 138.589265 51.549265) (width 0.2) (layer "F.Cu") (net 6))
 (segment (start 143.23 50.45) (end 143.2545 50.4255) (width 0.2) (layer "F.Cu") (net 6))
 (segment (start 138.589265 51.549265) (end 139.420735 51.549265) (width 0.2) (layer "F.Cu") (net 6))
 (segment (start 142.93 50.45) (end 143.23 50.45) (width 0.2) (layer "F.Cu") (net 6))
 (segment (start 143.2545 50.4255) (end 145.215 50.4255) (width 0.2) (layer "F.Cu") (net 6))
 (segment (start 131.38 51) (end 138.04 51) (width 0.2) (layer "F.Cu") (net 6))
 (segment (start 131.38 52.570002) (end 131.38 51) (width 0.2) (layer "F.Cu") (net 6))
 (segment (start 131.439998 52.63) (end 131.38 52.570002) (width 0.2) (layer "F.Cu") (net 6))
 (via (at 142.93 50.45) (size 0.6) (drill 0.3) (layers "F.Cu" "B.Cu") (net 6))
 (via (at 139.420735 51.549265) (size 0.6) (drill 0.3) (layers "F.Cu" "B.Cu") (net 6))
 (segment (start 140.52 50.45) (end 142.93 50.45) (width 0.2) (layer "B.Cu") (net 6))
 (segment (start 139.420735 51.549265) (end 140.52 50.45) (width 0.2) (layer "B.Cu") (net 6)))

